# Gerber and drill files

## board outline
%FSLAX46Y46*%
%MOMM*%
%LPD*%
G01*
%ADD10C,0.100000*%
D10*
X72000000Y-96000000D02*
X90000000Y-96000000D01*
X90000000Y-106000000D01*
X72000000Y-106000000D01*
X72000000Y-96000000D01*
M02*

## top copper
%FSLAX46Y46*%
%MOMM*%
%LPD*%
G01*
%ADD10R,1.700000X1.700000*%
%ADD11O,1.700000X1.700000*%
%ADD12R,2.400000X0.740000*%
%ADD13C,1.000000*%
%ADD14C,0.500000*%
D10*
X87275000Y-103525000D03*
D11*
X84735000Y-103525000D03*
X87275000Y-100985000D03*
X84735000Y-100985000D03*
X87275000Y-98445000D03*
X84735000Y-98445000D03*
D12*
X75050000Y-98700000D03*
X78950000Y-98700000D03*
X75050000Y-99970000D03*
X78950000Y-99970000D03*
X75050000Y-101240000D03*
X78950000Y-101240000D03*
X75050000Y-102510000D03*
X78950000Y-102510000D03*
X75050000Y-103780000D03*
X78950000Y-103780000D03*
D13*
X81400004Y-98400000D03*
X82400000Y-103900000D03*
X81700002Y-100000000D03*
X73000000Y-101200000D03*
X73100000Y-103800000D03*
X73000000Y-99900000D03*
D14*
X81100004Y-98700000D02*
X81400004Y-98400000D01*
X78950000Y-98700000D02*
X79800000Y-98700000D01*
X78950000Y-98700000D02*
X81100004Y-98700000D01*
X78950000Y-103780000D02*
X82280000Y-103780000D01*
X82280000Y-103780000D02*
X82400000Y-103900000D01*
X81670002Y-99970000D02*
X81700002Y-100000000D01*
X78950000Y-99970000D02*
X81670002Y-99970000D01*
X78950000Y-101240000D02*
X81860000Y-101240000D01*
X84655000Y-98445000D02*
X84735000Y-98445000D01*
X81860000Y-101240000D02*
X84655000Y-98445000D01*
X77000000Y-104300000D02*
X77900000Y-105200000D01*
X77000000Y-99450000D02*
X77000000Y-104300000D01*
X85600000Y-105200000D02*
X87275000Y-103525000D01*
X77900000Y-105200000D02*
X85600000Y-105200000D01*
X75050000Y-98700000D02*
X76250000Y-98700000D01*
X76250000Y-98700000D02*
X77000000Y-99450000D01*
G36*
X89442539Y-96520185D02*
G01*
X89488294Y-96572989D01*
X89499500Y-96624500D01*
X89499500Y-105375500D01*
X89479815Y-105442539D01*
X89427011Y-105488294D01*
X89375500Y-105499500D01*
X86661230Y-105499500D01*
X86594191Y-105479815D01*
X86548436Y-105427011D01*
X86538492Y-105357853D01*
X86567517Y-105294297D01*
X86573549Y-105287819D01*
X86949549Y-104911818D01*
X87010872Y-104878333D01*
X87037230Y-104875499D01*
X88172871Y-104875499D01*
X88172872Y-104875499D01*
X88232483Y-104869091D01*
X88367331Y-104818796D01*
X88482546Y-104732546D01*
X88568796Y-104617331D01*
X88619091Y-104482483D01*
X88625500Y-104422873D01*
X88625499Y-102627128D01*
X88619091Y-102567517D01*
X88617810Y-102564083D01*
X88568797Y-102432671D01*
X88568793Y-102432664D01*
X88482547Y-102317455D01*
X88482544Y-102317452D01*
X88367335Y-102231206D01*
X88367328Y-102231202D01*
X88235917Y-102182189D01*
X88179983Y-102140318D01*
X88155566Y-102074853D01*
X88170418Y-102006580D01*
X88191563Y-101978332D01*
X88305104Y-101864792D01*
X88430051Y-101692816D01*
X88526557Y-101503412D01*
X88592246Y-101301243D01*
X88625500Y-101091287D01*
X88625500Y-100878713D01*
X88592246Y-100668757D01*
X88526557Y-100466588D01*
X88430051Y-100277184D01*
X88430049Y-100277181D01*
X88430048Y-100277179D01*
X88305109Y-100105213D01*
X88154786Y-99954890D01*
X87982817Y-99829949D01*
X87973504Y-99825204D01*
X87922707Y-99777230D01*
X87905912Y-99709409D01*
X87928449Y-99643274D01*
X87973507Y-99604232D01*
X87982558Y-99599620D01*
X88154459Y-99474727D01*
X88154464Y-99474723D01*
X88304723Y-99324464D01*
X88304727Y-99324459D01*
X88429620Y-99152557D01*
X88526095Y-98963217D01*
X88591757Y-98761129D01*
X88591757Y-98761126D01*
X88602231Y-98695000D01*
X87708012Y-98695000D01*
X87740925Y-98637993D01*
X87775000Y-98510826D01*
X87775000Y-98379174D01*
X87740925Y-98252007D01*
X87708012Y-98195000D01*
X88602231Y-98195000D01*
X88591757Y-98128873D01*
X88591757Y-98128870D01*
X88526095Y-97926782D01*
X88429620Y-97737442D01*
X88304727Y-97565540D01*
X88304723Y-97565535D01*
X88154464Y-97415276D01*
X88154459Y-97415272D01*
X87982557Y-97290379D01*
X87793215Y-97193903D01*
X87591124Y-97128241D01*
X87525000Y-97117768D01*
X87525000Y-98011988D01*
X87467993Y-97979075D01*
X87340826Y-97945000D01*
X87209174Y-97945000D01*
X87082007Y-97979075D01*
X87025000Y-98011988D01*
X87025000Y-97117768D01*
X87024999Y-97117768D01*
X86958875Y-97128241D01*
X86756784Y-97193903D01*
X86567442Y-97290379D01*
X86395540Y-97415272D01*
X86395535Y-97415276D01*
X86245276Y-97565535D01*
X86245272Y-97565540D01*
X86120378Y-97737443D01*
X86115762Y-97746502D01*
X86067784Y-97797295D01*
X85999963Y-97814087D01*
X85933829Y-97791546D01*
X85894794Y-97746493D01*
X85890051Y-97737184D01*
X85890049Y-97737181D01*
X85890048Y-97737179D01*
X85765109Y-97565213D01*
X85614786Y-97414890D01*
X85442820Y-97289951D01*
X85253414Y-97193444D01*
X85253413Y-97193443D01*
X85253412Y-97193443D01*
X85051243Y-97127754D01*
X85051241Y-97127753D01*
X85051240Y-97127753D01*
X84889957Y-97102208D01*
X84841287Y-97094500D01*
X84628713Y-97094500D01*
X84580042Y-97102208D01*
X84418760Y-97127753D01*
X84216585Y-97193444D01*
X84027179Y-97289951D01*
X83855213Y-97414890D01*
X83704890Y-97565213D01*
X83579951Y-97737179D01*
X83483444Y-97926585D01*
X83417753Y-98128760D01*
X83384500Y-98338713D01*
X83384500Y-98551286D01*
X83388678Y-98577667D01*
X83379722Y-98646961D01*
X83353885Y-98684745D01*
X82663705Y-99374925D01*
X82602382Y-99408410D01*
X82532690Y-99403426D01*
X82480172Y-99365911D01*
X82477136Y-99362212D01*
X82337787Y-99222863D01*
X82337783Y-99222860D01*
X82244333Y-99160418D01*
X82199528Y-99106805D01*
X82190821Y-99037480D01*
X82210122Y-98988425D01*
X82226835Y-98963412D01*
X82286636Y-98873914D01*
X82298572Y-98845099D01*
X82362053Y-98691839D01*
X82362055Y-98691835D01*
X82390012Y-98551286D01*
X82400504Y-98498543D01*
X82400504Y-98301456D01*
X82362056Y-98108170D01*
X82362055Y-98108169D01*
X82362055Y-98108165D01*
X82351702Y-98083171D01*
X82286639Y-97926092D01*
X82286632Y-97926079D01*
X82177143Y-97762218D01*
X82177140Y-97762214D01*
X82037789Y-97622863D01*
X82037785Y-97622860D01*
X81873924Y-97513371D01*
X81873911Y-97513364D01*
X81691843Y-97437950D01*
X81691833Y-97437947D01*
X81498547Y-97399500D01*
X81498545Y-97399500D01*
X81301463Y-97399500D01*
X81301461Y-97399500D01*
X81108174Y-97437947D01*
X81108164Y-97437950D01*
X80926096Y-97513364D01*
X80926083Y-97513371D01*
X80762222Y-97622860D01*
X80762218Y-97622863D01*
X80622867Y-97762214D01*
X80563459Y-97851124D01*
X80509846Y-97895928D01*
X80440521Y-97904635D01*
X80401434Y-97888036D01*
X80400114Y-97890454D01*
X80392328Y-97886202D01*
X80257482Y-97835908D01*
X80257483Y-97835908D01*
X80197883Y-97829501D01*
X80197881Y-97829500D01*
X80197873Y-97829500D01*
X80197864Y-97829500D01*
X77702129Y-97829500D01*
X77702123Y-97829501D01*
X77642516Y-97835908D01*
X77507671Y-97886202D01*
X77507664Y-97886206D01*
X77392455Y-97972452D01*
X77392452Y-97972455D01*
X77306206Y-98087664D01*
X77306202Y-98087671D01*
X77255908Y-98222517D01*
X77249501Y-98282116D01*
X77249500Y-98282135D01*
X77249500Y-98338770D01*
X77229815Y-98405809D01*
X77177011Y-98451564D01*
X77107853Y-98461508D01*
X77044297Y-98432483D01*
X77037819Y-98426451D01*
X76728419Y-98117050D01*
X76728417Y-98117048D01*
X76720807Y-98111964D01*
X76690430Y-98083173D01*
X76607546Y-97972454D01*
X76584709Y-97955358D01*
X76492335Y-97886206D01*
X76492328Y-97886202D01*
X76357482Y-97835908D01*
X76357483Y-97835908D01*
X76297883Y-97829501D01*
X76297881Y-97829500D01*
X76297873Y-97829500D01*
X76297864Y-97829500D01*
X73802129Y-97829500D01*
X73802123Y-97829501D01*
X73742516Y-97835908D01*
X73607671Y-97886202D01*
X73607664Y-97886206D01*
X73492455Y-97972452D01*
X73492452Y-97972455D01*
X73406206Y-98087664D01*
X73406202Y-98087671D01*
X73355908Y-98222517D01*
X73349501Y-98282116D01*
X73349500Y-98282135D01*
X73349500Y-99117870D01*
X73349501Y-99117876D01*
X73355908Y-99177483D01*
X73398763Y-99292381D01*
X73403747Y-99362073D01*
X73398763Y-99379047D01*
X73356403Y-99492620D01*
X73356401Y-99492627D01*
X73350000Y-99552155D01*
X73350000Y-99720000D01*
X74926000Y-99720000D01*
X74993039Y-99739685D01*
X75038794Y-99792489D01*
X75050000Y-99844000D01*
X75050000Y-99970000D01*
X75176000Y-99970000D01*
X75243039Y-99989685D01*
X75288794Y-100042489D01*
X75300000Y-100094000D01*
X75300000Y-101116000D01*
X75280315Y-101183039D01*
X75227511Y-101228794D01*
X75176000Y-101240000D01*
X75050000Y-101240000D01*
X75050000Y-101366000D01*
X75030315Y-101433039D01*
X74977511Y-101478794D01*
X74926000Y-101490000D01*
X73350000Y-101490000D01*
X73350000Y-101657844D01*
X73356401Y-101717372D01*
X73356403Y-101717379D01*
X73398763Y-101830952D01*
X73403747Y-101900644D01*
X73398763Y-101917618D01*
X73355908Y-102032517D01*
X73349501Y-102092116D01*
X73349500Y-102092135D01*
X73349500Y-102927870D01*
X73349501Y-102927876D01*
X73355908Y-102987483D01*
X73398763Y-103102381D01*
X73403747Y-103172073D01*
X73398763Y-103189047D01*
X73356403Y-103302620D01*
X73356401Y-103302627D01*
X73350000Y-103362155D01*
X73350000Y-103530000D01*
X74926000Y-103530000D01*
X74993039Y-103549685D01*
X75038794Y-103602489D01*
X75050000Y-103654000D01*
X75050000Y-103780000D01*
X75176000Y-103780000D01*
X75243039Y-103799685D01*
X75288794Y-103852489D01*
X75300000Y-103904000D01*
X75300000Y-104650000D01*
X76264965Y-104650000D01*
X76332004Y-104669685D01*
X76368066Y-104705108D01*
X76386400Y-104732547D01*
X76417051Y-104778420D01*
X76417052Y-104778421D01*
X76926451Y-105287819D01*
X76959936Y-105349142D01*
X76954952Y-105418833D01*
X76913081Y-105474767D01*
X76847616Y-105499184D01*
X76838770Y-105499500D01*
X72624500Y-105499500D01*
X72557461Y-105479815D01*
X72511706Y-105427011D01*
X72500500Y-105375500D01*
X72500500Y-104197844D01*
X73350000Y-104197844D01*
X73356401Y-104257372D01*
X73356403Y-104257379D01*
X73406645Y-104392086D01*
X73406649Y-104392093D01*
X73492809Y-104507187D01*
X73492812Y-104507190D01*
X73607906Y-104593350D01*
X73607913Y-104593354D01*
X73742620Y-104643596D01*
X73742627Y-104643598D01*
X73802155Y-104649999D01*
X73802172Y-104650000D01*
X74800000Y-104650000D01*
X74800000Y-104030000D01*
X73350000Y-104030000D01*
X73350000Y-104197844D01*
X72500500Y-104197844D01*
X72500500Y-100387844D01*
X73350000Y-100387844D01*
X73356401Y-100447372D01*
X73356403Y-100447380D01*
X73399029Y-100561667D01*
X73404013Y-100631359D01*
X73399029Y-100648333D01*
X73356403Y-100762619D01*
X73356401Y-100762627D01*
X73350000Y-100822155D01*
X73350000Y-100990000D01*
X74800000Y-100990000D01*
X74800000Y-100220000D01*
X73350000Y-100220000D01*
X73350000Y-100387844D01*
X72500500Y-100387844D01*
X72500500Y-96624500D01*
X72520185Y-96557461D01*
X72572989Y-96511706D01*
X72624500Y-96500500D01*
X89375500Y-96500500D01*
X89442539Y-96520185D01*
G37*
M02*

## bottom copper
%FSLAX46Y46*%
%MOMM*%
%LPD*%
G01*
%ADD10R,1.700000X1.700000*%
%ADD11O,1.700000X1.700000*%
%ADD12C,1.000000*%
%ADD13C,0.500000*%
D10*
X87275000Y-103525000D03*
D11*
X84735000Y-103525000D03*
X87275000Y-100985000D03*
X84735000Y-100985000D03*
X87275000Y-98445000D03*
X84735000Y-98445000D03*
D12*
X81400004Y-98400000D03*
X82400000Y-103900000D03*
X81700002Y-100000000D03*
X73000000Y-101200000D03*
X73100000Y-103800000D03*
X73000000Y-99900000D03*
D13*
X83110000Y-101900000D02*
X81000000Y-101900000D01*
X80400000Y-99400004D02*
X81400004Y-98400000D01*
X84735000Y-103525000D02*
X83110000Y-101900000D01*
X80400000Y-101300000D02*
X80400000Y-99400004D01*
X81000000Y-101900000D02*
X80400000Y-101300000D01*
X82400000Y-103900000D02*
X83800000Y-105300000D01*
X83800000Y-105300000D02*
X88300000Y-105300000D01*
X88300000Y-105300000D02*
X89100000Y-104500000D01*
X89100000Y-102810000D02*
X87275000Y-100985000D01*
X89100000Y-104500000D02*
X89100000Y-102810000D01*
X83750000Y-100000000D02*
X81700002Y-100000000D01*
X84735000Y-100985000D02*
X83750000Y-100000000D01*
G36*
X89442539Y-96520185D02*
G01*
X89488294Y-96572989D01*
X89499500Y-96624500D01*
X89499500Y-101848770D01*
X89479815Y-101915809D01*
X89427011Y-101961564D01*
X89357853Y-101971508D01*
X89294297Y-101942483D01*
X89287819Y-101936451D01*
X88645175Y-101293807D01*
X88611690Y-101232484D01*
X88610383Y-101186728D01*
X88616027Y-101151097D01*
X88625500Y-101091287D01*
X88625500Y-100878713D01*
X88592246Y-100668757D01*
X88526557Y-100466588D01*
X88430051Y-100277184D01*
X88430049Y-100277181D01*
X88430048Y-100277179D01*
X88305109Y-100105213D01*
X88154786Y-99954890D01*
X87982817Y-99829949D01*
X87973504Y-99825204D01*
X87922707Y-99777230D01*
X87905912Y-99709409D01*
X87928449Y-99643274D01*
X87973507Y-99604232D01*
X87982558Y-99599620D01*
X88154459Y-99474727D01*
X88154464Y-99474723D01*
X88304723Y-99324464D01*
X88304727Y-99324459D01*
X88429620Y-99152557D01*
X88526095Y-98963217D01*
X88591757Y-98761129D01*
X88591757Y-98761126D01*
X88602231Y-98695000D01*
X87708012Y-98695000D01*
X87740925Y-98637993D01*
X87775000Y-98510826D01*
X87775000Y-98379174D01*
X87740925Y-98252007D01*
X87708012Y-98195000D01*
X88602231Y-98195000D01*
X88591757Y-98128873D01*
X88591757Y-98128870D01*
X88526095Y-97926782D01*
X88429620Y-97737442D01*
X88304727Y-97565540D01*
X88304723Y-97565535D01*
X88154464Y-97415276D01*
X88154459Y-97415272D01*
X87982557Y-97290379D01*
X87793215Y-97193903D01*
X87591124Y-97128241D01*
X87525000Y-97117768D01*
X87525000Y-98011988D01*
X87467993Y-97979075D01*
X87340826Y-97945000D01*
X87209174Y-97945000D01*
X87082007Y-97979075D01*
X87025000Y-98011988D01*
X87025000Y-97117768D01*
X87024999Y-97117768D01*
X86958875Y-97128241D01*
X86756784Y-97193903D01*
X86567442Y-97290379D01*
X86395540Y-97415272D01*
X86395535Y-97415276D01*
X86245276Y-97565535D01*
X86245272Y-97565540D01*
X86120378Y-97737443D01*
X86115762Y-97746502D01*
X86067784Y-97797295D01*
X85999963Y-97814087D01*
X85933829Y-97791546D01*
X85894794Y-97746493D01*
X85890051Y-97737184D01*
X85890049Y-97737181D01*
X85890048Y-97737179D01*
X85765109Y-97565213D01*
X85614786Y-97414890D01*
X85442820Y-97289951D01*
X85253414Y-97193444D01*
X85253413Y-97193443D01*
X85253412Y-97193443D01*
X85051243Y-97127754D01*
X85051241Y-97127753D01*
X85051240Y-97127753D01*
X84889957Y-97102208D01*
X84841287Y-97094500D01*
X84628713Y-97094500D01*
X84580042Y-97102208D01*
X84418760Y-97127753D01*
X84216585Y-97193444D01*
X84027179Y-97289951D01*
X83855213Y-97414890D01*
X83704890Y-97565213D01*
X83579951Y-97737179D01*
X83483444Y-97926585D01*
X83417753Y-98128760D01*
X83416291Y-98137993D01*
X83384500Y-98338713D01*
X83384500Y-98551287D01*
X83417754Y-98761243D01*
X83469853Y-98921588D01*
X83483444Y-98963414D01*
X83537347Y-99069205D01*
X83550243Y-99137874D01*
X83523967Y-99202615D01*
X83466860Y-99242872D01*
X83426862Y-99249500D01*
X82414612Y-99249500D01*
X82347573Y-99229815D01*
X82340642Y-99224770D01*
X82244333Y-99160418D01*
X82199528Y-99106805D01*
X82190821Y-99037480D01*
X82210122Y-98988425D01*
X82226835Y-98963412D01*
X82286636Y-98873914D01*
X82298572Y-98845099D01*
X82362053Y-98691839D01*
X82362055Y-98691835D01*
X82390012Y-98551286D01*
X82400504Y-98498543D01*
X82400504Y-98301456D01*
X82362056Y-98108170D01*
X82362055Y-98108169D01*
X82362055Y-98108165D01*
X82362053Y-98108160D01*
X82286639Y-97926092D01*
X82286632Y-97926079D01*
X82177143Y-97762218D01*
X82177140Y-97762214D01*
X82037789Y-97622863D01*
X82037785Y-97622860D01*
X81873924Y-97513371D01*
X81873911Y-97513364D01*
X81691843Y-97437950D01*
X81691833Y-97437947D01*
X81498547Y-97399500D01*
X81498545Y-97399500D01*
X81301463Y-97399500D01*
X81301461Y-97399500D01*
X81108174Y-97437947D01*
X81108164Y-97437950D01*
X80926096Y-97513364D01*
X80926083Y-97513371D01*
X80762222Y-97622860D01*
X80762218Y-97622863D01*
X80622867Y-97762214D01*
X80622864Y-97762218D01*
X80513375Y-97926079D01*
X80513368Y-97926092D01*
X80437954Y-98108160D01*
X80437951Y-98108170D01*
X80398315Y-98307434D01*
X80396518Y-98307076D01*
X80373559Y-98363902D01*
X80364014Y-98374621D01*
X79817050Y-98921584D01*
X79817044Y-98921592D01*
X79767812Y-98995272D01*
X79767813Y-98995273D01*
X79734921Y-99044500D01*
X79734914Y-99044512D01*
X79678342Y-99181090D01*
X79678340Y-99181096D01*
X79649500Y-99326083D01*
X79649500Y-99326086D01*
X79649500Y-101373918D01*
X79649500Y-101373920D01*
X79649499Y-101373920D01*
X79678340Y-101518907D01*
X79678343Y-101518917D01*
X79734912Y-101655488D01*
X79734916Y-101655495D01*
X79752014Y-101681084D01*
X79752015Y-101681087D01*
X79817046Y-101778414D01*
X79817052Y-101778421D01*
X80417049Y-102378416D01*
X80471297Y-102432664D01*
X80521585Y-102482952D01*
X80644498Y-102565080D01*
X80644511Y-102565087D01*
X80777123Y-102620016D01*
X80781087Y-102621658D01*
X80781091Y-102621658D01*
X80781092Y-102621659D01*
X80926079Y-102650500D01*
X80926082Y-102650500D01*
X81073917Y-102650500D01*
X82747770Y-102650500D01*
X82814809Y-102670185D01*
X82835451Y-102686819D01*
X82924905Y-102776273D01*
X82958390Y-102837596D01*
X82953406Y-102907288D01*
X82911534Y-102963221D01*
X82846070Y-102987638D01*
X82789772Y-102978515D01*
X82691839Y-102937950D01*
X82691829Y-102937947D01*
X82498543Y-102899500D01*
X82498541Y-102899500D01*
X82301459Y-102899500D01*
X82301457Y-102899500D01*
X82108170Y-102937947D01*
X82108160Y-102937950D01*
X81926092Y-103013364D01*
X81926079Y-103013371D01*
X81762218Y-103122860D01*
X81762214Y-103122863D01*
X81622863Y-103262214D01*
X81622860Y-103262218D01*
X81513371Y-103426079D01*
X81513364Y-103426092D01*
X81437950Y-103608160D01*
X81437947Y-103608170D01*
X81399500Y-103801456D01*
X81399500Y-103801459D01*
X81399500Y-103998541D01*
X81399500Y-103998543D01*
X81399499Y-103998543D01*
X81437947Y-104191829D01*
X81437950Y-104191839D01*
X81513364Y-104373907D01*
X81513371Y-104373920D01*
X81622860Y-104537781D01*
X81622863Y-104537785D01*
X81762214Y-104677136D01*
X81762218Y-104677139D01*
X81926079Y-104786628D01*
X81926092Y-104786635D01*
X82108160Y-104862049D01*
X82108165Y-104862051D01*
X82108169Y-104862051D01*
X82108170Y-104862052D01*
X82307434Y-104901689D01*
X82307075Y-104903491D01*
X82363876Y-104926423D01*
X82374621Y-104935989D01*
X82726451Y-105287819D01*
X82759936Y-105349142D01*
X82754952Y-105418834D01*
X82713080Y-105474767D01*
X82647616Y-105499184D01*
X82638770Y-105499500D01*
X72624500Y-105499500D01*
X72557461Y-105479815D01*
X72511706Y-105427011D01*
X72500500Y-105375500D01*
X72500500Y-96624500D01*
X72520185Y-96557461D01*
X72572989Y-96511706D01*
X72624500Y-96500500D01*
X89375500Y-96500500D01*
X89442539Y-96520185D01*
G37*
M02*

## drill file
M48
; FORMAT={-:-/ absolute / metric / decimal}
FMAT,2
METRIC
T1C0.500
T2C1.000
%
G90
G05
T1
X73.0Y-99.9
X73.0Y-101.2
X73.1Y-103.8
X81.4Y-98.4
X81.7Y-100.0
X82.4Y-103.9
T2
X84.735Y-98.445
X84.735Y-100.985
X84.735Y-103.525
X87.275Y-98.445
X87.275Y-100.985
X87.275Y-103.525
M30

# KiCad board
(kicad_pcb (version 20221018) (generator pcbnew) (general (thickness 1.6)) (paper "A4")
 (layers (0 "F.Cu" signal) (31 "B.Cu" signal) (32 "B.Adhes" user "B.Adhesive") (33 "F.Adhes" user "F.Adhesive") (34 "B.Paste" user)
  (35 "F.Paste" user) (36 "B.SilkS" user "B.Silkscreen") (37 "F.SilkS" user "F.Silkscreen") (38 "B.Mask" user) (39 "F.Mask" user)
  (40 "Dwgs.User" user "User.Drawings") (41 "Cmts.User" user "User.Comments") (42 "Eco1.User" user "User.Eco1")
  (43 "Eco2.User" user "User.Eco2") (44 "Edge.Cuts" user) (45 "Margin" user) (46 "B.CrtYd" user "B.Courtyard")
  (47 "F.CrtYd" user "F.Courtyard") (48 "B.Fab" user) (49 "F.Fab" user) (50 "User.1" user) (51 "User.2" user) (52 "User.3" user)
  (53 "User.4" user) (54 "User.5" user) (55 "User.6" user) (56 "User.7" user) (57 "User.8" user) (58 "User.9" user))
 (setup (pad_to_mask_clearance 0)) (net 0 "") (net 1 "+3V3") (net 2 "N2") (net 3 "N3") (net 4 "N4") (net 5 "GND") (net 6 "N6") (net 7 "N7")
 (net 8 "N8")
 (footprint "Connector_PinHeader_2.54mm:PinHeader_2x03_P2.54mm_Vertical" (layer "F.Cu") (at 87.275 103.525 180)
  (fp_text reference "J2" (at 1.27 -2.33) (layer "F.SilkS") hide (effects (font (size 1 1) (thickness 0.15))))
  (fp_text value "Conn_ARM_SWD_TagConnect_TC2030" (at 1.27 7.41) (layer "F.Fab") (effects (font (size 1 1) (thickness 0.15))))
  (pad "1" thru_hole rect (at 0 0 180) (size 1.7 1.7) (drill 1) (layers "*.Cu" "*.Mask") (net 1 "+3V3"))
  (pad "2" thru_hole oval (at 2.54 0 180) (size 1.7 1.7) (drill 1) (layers "*.Cu" "*.Mask") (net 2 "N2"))
  (pad "3" thru_hole oval (at 0 2.54 180) (size 1.7 1.7) (drill 1) (layers "*.Cu" "*.Mask") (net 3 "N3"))
  (pad "4" thru_hole oval (at 2.54 2.54 180) (size 1.7 1.7) (drill 1) (layers "*.Cu" "*.Mask") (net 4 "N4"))
  (pad "5" thru_hole oval (at 0 5.08 180) (size 1.7 1.7) (drill 1) (layers "*.Cu" "*.Mask") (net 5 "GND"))
  (pad "6" thru_hole oval (at 2.54 5.08 180) (size 1.7 1.7) (drill 1) (layers "*.Cu" "*.Mask") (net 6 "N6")))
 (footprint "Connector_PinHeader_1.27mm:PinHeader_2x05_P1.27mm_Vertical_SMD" (layer "F.Cu") (at 77 101.24)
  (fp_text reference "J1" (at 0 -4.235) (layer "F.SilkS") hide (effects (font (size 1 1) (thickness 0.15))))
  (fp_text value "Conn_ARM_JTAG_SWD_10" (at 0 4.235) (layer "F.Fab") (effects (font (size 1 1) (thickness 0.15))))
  (pad "1" smd rect (at -1.95 -2.54) (size 2.4 0.74) (layers "F.Cu" "F.Paste" "F.Mask") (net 1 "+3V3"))
  (pad "2" smd rect (at 1.95 -2.54) (size 2.4 0.74) (layers "F.Cu" "F.Paste" "F.Mask") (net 2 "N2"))
  (pad "3" smd rect (at -1.95 -1.27) (size 2.4 0.74) (layers "F.Cu" "F.Paste" "F.Mask") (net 5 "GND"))
  (pad "4" smd rect (at 1.95 -1.27) (size 2.4 0.74) (layers "F.Cu" "F.Paste" "F.Mask") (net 4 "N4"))
  (pad "5" smd rect (at -1.95 0) (size 2.4 0.74) (layers "F.Cu" "F.Paste" "F.Mask") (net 5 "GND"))
  (pad "6" smd rect (at 1.95 0) (size 2.4 0.74) (layers "F.Cu" "F.Paste" "F.Mask") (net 6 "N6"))
  (pad "7" smd rect (at -1.95 1.27) (size 2.4 0.74) (layers "F.Cu" "F.Paste" "F.Mask") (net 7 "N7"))
  (pad "8" smd rect (at 1.95 1.27) (size 2.4 0.74) (layers "F.Cu" "F.Paste" "F.Mask") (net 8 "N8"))
  (pad "9" smd rect (at -1.95 2.54) (size 2.4 0.74) (layers "F.Cu" "F.Paste" "F.Mask") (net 5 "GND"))
  (pad "10" smd rect (at 1.95 2.54) (size 2.4 0.74) (layers "F.Cu" "F.Paste" "F.Mask") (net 3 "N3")))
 (gr_rect (start 72 96) (end 90 106) (stroke (width 0.1) (type default)) (fill none) (layer "Edge.Cuts"))
 (segment (start 81.100004 98.7) (end 81.400004 98.4) (width 0.5) (layer "F.Cu") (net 2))
 (segment (start 78.95 98.7) (end 79.8 98.7) (width 0.5) (layer "F.Cu") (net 2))
 (segment (start 78.95 98.7) (end 81.100004 98.7) (width 0.5) (layer "F.Cu") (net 2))
 (via (at 81.400004 98.4) (size 1) (drill 0.5) (layers "F.Cu" "B.Cu") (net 2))
 (segment (start 83.11 101.9) (end 81 101.9) (width 0.5) (layer "B.Cu") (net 2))
 (segment (start 80.4 99.400004) (end 81.400004 98.4) (width 0.5) (layer "B.Cu") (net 2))
 (segment (start 84.735 103.525) (end 83.11 101.9) (width 0.5) (layer "B.Cu") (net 2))
 (segment (start 80.4 101.3) (end 80.4 99.400004) (width 0.5) (layer "B.Cu") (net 2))
 (segment (start 81 101.9) (end 80.4 101.3) (width 0.5) (layer "B.Cu") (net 2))
 (segment (start 78.95 103.78) (end 82.28 103.78) (width 0.5) (layer "F.Cu") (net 3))
 (segment (start 82.28 103.78) (end 82.4 103.9) (width 0.5) (layer "F.Cu") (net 3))
 (via (at 82.4 103.9) (size 1) (drill 0.5) (layers "F.Cu" "B.Cu") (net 3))
 (segment (start 82.4 103.9) (end 83.8 105.3) (width 0.5) (layer "B.Cu") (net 3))
 (segment (start 83.8 105.3) (end 88.3 105.3) (width 0.5) (layer "B.Cu") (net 3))
 (segment (start 88.3 105.3) (end 89.1 104.5) (width 0.5) (layer "B.Cu") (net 3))
 (segment (start 89.1 102.81) (end 87.275 100.985) (width 0.5) (layer "B.Cu") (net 3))
 (segment (start 89.1 104.5) (end 89.1 102.81) (width 0.5) (layer "B.Cu") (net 3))
 (segment (start 81.670002 99.97) (end 81.700002 100) (width 0.5) (layer "F.Cu") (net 4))
 (segment (start 78.95 99.97) (end 81.670002 99.97) (width 0.5) (layer "F.Cu") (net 4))
 (via (at 81.700002 100) (size 1) (drill 0.5) (layers "F.Cu" "B.Cu") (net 4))
 (segment (start 83.75 100) (end 81.700002 100) (width 0.5) (layer "B.Cu") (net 4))
 (segment (start 84.735 100.985) (end 83.75 100) (width 0.5) (layer "B.Cu") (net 4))
 (segment (start 78.95 101.24) (end 81.86 101.24) (width 0.5) (layer "F.Cu") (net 6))
 (segment (start 84.655 98.445) (end 84.735 98.445) (width 0.5) (layer "F.Cu") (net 6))
 (segment (start 81.86 101.24) (end 84.655 98.445) (width 0.5) (layer "F.Cu") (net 6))
 (segment (start 77 104.3) (end 77.9 105.2) (width 0.5) (layer "F.Cu") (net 1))
 (segment (start 77 99.45) (end 77 104.3) (width 0.5) (layer "F.Cu") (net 1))
 (segment (start 85.6 105.2) (end 87.275 103.525) (width 0.5) (layer "F.Cu") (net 1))
 (segment (start 77.9 105.2) (end 85.6 105.2) (width 0.5) (layer "F.Cu") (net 1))
 (segment (start 75.05 98.7) (end 76.25 98.7) (width 0.5) (layer "F.Cu") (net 1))
 (segment (start 76.25 98.7) (end 77 99.45) (width 0.5) (layer "F.Cu") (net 1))
 (via (at 73 101.2) (size 1) (drill 0.5) (layers "F.Cu" "B.Cu") (free) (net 5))
 (via (at 73.1 103.8) (size 1) (drill 0.5) (layers "F.Cu" "B.Cu") (free) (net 5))
 (via (at 73 99.9) (size 1) (drill 0.5) (layers "F.Cu" "B.Cu") (free) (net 5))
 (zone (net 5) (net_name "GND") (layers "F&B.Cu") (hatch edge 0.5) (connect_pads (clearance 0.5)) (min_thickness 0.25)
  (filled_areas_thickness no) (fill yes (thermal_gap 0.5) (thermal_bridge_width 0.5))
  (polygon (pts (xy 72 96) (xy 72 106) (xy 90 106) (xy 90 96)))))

